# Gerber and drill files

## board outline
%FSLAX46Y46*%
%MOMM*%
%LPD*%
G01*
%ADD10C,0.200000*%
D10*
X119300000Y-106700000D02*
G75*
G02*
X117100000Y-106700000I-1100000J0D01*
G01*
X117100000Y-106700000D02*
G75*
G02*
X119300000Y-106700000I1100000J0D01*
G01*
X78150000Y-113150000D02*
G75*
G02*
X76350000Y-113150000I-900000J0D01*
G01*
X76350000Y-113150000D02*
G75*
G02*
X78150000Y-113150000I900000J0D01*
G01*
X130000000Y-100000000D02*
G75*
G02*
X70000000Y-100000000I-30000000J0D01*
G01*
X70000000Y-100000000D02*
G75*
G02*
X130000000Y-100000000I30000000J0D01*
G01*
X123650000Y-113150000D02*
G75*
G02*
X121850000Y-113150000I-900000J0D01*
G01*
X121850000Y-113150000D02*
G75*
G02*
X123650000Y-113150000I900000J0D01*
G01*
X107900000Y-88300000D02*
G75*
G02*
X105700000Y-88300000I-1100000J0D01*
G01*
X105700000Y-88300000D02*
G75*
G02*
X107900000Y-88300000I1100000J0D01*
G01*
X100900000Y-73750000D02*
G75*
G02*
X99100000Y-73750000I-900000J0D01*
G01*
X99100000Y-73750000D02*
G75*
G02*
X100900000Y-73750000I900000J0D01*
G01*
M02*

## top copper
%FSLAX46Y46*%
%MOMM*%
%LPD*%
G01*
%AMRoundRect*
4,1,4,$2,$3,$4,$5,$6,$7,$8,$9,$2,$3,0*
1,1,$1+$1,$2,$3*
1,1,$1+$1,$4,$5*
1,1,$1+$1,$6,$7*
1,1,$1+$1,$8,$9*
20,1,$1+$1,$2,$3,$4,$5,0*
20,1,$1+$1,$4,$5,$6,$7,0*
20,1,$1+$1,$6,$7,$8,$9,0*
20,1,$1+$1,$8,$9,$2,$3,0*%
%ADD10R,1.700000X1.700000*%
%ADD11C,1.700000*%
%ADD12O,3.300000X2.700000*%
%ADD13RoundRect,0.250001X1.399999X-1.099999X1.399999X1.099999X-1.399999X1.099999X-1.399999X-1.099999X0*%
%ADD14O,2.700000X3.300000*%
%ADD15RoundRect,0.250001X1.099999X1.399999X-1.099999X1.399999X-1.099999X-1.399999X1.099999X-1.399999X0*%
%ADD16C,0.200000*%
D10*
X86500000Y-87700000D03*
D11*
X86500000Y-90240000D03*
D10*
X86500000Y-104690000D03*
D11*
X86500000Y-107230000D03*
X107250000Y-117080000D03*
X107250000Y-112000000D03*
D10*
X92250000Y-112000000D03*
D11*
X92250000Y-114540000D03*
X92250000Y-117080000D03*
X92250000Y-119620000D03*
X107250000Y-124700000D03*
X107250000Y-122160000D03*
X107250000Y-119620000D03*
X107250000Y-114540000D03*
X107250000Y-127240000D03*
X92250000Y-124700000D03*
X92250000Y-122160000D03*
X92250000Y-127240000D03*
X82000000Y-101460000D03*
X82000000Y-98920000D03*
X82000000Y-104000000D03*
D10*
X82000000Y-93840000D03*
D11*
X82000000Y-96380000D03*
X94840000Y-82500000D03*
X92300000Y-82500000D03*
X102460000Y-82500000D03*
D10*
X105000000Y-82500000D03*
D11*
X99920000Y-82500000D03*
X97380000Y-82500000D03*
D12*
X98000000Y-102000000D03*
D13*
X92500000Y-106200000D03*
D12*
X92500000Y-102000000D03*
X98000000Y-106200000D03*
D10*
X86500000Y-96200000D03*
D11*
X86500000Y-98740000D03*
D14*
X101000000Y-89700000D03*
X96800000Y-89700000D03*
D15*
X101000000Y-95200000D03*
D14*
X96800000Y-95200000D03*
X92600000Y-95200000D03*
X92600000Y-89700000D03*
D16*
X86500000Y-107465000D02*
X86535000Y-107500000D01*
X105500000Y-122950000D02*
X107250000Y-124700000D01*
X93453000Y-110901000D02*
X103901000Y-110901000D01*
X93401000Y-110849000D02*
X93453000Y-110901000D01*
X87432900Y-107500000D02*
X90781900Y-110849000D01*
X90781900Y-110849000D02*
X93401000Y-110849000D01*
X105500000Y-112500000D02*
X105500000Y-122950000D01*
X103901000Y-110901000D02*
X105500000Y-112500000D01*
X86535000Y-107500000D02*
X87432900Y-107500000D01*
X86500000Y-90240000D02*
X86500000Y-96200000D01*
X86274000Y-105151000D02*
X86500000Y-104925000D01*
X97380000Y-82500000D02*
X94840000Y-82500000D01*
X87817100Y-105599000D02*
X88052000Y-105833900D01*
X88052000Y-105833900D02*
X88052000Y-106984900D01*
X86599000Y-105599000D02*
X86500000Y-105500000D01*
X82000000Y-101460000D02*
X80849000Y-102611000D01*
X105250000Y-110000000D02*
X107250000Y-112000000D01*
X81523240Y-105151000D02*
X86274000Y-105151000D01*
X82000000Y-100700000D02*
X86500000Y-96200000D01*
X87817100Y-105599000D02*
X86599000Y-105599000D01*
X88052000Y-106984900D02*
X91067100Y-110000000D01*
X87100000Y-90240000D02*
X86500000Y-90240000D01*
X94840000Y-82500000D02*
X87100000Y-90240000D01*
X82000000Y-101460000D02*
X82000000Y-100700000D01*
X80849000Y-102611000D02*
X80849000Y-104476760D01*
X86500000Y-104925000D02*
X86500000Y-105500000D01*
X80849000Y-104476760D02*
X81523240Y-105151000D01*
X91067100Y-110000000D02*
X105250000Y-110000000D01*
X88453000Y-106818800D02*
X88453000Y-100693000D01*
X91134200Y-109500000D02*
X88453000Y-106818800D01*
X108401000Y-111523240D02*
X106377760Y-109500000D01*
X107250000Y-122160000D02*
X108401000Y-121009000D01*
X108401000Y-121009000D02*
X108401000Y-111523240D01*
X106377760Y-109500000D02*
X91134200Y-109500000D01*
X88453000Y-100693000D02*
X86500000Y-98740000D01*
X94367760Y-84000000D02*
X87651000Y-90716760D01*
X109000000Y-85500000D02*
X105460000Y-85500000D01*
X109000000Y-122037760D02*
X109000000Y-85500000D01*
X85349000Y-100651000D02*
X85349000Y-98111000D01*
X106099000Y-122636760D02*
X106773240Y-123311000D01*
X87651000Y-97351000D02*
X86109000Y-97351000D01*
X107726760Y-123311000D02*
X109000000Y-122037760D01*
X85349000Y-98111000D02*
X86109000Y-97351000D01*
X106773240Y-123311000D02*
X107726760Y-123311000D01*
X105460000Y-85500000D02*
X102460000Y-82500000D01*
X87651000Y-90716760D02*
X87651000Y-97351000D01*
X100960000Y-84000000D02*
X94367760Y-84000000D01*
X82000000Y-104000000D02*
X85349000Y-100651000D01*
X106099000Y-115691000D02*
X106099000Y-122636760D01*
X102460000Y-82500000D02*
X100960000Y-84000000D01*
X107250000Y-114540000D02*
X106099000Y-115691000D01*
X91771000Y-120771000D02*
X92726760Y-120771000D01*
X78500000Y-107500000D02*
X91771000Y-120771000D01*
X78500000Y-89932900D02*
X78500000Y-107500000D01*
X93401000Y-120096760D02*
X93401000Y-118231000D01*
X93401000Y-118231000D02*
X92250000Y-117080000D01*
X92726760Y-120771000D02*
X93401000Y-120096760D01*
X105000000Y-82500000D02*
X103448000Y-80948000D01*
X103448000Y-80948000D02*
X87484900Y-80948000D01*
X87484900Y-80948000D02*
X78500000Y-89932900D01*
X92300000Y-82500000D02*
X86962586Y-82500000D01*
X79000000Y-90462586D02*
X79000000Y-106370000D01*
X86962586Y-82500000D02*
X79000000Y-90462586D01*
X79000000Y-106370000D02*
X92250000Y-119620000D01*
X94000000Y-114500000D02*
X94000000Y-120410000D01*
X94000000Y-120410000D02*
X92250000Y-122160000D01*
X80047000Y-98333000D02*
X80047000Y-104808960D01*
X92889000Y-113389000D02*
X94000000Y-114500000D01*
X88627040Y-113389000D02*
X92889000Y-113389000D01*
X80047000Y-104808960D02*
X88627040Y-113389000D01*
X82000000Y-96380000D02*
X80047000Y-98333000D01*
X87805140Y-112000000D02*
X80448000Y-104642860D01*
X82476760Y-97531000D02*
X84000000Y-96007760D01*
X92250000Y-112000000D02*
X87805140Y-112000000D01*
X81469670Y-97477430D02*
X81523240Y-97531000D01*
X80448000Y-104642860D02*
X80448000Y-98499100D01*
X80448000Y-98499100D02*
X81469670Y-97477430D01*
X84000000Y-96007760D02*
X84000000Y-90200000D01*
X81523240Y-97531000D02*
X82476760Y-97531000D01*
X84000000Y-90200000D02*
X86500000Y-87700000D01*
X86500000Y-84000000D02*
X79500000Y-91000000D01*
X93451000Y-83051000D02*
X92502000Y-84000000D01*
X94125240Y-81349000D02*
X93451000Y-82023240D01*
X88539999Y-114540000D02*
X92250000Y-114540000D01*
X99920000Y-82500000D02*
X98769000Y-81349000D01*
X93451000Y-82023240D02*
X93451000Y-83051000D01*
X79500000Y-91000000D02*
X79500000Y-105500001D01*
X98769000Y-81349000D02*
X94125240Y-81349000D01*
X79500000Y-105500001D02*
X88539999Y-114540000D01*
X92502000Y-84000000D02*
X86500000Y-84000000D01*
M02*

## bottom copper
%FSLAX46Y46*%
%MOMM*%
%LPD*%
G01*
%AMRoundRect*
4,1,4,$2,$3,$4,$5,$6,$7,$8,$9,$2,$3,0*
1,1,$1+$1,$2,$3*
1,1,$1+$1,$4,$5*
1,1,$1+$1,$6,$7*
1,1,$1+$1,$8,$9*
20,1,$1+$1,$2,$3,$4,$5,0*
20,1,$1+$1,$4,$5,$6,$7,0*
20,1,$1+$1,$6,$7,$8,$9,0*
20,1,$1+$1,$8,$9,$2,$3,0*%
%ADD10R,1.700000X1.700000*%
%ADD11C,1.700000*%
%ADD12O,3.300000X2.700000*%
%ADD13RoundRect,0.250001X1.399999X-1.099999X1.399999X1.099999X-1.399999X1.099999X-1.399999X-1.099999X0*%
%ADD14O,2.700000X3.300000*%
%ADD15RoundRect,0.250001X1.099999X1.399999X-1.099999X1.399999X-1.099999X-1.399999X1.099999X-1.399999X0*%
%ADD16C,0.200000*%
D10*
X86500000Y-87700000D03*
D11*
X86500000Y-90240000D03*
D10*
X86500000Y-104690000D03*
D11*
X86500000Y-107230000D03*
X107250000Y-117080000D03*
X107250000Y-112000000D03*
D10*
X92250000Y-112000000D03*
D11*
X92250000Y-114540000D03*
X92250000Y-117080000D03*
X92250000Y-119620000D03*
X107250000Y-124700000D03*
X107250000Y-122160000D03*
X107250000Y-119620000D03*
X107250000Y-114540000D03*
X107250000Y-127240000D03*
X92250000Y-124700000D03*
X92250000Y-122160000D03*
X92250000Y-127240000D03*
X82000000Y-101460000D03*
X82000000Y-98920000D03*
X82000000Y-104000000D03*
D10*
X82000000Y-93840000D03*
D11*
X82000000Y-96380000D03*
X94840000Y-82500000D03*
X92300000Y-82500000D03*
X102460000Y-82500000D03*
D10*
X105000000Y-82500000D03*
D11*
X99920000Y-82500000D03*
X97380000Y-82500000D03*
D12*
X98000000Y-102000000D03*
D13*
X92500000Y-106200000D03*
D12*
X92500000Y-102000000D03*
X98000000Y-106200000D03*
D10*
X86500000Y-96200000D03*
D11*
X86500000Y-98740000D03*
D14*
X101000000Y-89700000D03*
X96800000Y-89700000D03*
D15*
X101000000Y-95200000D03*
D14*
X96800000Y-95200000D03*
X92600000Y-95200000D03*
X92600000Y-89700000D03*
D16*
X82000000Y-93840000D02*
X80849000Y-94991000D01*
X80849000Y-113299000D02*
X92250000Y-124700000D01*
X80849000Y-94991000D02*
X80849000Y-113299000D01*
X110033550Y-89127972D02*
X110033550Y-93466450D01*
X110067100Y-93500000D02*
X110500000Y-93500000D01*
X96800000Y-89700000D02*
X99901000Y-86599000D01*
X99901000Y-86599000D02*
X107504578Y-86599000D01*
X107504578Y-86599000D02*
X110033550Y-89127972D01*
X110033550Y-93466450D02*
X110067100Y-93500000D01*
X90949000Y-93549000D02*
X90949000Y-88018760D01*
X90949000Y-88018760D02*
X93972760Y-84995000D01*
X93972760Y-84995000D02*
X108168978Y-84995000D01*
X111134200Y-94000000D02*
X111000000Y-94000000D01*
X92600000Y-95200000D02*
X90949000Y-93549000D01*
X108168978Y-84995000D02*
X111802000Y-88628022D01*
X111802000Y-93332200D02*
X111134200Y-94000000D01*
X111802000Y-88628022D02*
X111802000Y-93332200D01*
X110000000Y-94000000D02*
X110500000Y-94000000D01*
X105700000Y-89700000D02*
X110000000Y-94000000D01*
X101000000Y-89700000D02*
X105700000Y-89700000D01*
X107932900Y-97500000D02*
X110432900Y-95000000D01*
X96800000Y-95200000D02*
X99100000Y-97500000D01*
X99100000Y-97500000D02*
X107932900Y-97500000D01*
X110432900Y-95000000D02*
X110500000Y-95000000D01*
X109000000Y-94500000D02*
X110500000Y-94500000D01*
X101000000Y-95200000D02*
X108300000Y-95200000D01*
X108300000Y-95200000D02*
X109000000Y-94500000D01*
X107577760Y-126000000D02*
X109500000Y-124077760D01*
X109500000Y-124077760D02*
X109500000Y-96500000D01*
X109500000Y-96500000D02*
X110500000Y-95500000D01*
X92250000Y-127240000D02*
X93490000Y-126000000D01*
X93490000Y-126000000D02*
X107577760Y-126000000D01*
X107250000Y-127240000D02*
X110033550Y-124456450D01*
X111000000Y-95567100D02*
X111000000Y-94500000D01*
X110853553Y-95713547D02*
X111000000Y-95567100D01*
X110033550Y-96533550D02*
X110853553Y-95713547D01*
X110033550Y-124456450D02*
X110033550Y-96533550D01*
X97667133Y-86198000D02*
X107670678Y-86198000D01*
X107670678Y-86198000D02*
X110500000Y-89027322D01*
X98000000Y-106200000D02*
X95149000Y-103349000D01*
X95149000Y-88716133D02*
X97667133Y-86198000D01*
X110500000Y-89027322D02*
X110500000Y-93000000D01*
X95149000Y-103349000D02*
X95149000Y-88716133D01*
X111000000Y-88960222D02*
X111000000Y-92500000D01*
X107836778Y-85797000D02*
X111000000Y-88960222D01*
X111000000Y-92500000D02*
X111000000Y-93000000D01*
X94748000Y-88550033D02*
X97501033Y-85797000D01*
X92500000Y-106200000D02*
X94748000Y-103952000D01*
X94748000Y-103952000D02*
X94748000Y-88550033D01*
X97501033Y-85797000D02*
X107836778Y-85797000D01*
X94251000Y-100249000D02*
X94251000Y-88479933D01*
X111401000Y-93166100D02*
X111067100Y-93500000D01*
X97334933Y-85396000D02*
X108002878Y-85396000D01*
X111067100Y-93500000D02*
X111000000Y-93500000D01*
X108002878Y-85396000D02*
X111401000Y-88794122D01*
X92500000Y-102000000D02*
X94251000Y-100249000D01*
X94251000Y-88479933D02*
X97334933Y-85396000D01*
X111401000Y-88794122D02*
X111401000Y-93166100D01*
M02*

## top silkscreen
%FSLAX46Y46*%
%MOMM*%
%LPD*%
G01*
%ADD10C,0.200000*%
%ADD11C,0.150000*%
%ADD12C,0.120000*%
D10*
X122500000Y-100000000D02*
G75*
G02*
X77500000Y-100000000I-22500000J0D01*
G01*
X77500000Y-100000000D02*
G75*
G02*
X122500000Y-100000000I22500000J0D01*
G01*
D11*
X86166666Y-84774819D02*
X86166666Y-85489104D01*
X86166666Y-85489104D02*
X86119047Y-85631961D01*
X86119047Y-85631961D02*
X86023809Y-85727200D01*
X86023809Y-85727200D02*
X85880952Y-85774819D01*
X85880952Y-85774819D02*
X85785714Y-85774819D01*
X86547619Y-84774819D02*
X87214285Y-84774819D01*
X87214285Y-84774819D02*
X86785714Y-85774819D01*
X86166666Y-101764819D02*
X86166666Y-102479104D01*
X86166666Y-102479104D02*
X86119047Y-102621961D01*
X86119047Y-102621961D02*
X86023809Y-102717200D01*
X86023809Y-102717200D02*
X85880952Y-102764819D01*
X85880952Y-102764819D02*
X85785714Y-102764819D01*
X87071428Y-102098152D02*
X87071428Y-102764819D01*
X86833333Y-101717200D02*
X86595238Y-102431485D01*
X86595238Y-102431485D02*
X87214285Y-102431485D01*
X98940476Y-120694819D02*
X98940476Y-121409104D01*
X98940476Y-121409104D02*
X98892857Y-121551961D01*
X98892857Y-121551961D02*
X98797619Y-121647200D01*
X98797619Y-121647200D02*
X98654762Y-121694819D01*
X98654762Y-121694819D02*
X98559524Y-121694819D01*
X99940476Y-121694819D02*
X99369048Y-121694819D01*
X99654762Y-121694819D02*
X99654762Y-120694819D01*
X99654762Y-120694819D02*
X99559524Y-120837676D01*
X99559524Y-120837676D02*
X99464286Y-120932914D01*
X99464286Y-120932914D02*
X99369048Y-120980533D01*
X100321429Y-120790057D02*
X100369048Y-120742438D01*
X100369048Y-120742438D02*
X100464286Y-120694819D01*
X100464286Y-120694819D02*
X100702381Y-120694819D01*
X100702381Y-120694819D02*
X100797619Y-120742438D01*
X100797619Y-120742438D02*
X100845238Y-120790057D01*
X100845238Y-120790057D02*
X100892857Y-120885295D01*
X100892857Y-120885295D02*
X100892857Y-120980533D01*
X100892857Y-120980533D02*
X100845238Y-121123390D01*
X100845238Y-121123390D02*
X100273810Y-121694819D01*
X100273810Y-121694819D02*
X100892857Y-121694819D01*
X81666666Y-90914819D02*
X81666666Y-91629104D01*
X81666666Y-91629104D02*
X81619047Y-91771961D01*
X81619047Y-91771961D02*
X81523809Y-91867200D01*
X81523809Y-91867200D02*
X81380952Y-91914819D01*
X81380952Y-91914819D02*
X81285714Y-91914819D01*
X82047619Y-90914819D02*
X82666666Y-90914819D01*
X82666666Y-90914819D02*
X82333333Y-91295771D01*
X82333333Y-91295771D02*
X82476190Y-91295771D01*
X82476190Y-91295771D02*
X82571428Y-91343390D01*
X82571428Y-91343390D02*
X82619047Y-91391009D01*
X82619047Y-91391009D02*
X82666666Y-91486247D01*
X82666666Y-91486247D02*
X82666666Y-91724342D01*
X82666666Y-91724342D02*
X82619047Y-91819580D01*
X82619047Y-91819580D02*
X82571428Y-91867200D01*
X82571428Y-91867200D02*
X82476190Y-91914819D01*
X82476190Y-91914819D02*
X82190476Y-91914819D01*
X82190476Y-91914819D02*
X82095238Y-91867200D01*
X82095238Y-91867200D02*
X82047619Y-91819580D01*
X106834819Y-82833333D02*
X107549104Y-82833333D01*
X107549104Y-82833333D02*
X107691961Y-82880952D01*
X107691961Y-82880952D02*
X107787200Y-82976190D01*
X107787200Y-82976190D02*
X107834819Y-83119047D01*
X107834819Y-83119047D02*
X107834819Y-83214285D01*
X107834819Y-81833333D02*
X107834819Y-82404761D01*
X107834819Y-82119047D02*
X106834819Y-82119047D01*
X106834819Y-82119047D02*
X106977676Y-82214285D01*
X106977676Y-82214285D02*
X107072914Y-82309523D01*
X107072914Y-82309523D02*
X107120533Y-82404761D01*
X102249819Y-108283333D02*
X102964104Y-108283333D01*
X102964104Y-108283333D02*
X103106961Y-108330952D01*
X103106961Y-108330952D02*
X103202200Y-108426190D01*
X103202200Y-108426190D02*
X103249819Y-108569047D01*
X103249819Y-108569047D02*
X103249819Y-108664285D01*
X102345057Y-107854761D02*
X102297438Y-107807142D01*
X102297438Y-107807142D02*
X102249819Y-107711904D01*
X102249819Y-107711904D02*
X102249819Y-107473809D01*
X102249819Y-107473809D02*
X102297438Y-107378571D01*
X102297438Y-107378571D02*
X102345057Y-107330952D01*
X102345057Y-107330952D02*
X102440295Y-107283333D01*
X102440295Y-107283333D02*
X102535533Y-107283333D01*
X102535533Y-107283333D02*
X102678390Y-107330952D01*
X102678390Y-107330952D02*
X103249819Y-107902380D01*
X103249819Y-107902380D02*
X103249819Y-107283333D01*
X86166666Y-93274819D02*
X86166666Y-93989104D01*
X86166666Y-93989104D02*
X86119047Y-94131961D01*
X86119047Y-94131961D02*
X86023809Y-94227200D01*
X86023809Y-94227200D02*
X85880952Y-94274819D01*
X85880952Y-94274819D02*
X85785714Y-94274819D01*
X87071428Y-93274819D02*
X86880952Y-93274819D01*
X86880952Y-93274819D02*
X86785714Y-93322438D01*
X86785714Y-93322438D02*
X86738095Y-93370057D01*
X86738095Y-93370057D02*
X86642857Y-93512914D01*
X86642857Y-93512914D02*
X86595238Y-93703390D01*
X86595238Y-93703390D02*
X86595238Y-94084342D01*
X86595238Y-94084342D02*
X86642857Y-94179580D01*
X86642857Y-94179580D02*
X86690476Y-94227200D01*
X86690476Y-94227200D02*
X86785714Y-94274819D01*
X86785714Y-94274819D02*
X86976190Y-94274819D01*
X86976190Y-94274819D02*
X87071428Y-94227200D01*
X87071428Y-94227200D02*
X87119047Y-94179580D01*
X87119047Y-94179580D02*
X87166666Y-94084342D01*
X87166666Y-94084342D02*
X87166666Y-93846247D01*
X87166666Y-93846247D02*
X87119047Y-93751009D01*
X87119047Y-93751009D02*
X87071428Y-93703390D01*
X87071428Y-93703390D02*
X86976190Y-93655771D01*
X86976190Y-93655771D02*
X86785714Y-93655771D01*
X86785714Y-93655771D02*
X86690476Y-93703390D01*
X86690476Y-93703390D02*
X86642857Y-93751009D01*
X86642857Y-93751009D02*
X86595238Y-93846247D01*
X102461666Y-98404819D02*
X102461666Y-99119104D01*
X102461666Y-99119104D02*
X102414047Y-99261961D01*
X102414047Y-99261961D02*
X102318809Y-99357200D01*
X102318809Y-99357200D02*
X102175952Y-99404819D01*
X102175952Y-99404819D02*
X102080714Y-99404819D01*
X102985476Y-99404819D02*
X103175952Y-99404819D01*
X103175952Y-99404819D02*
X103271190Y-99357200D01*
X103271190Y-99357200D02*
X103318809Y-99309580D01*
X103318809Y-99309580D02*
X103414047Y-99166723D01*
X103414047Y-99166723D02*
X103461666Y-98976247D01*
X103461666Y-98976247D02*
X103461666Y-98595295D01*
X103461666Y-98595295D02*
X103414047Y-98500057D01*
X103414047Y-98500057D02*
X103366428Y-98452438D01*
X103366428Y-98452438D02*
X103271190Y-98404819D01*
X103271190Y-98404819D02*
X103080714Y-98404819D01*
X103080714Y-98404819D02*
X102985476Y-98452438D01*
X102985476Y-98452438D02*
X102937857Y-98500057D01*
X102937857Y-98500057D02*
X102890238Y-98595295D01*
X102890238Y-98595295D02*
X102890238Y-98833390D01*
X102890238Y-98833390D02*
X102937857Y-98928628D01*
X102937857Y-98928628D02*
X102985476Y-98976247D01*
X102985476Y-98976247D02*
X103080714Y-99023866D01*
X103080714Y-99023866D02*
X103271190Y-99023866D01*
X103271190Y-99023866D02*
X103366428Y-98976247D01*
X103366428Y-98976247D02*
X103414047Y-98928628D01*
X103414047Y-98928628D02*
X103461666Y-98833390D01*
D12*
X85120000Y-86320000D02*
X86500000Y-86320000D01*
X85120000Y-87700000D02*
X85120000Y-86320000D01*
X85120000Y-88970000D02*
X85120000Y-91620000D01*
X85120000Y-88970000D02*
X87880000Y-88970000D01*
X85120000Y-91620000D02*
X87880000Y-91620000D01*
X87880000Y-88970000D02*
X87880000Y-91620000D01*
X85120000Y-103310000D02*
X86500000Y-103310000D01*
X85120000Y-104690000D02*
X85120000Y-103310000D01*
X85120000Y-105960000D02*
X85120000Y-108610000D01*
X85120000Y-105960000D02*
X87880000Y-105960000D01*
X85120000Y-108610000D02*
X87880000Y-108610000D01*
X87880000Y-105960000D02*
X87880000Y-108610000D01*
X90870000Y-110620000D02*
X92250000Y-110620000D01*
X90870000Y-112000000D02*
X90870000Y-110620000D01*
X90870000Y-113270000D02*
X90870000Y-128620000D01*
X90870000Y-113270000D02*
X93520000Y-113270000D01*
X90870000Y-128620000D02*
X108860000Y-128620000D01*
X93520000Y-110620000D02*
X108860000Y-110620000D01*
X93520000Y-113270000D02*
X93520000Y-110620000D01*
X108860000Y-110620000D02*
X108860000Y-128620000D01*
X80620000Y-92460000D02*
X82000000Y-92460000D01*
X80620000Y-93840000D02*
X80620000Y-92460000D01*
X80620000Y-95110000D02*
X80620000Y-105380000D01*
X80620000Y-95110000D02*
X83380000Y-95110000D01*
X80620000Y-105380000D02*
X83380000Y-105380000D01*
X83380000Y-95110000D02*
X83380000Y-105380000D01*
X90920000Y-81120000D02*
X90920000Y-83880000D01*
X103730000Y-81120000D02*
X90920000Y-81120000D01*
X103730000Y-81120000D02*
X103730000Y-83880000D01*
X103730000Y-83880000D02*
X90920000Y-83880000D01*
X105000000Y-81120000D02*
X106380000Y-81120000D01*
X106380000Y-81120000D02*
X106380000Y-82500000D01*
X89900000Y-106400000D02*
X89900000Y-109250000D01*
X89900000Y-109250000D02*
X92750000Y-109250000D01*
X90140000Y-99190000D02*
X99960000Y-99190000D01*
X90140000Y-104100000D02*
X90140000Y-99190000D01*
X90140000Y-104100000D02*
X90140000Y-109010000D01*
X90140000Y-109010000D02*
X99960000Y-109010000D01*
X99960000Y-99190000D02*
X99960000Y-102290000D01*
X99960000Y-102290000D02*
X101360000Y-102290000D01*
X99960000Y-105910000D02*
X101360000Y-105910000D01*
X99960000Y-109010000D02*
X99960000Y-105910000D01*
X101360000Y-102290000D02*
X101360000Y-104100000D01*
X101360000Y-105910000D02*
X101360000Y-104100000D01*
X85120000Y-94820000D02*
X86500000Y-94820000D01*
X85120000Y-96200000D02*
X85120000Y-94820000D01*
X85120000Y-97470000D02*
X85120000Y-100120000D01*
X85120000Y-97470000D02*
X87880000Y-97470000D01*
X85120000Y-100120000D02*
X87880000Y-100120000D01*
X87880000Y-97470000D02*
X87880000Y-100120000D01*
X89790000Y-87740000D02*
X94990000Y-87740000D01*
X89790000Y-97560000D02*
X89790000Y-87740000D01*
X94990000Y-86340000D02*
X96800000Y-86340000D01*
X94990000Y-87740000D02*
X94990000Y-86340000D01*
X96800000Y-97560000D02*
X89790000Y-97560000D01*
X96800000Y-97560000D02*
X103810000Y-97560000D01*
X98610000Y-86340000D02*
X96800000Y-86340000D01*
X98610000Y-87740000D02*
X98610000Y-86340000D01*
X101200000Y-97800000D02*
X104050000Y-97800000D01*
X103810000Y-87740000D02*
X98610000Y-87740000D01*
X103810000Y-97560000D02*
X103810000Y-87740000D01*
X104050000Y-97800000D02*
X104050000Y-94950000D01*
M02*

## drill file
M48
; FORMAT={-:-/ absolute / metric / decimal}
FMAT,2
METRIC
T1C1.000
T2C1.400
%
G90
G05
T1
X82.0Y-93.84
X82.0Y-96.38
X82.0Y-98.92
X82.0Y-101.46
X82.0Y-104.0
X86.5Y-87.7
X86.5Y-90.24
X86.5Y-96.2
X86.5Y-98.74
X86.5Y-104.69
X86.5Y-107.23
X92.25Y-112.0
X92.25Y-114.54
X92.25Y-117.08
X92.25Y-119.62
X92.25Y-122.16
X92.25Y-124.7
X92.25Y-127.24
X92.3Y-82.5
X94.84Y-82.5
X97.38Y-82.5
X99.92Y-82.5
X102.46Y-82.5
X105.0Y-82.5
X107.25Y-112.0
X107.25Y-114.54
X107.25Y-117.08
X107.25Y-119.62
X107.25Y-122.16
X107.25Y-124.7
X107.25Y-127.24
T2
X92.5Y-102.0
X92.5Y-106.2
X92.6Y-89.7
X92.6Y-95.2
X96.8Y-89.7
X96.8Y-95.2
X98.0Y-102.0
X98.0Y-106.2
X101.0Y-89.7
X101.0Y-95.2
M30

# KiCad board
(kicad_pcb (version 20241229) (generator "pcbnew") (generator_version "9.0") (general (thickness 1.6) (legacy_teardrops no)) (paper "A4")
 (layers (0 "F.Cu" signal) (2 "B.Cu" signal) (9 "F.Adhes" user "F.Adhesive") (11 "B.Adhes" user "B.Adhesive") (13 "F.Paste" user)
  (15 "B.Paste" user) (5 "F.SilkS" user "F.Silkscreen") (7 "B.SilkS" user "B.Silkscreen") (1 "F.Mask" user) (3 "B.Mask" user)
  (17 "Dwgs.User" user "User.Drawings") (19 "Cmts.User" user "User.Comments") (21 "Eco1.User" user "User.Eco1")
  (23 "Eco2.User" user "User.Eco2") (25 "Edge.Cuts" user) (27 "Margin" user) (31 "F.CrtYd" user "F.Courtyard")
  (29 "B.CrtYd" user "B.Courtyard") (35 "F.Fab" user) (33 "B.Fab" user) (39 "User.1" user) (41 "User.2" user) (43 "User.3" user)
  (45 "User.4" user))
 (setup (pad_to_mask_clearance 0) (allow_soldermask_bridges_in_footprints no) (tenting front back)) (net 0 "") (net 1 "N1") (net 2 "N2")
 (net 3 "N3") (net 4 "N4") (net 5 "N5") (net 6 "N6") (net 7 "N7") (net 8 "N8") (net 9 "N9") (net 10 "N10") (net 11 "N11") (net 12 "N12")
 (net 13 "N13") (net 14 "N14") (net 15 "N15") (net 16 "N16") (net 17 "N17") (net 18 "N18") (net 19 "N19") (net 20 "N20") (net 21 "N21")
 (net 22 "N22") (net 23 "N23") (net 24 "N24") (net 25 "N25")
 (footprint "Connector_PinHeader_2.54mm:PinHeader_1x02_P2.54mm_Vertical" (layer "F.Cu") (at 86.5 87.7)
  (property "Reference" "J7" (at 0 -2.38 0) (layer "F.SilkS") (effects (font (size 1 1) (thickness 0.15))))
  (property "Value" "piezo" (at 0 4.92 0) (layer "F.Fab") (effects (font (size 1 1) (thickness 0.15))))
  (fp_line (start -1.38 -1.38) (end 0 -1.38) (stroke (width 0.12) (type solid)) (layer "F.SilkS"))
  (fp_line (start -1.38 0) (end -1.38 -1.38) (stroke (width 0.12) (type solid)) (layer "F.SilkS"))
  (fp_line (start -1.38 1.27) (end -1.38 3.92) (stroke (width 0.12) (type solid)) (layer "F.SilkS"))
  (fp_line (start -1.38 1.27) (end 1.38 1.27) (stroke (width 0.12) (type solid)) (layer "F.SilkS"))
  (fp_line (start -1.38 3.92) (end 1.38 3.92) (stroke (width 0.12) (type solid)) (layer "F.SilkS"))
  (fp_line (start 1.38 1.27) (end 1.38 3.92) (stroke (width 0.12) (type solid)) (layer "F.SilkS"))
  (pad "1" thru_hole rect (at 0 0) (size 1.7 1.7) (drill 1) (layers "*.Cu" "*.Mask") (remove_unused_layers no) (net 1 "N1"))
  (pad "2" thru_hole circle (at 0 2.54) (size 1.7 1.7) (drill 1) (layers "*.Cu" "*.Mask") (remove_unused_layers no) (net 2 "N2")))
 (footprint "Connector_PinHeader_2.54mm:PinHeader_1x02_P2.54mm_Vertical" (layer "F.Cu") (at 86.5 104.69)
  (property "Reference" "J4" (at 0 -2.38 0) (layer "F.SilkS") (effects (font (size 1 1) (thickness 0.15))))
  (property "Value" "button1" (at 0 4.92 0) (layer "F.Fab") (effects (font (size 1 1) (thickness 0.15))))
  (fp_line (start -1.38 -1.38) (end 0 -1.38) (stroke (width 0.12) (type solid)) (layer "F.SilkS"))
  (fp_line (start -1.38 0) (end -1.38 -1.38) (stroke (width 0.12) (type solid)) (layer "F.SilkS"))
  (fp_line (start -1.38 1.27) (end -1.38 3.92) (stroke (width 0.12) (type solid)) (layer "F.SilkS"))
  (fp_line (start -1.38 1.27) (end 1.38 1.27) (stroke (width 0.12) (type solid)) (layer "F.SilkS"))
  (fp_line (start -1.38 3.92) (end 1.38 3.92) (stroke (width 0.12) (type solid)) (layer "F.SilkS"))
  (fp_line (start 1.38 1.27) (end 1.38 3.92) (stroke (width 0.12) (type solid)) (layer "F.SilkS"))
  (pad "1" thru_hole rect (at 0 0) (size 1.7 1.7) (drill 1) (layers "*.Cu" "*.Mask") (remove_unused_layers no) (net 2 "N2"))
  (pad "2" thru_hole circle (at 0 2.54) (size 1.7 1.7) (drill 1) (layers "*.Cu" "*.Mask") (remove_unused_layers no) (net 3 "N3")))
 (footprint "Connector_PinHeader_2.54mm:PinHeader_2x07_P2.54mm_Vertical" (layer "F.Cu") (at 92.25 112)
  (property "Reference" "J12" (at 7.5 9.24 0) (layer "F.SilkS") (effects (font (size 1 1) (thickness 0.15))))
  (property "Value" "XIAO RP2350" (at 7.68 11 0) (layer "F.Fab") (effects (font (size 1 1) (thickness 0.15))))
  (fp_line (start -1.38 -1.38) (end 0 -1.38) (stroke (width 0.12) (type solid)) (layer "F.SilkS"))
  (fp_line (start -1.38 0) (end -1.38 -1.38) (stroke (width 0.12) (type solid)) (layer "F.SilkS"))
  (fp_line (start -1.38 1.27) (end -1.38 16.62) (stroke (width 0.12) (type solid)) (layer "F.SilkS"))
  (fp_line (start -1.38 1.27) (end 1.27 1.27) (stroke (width 0.12) (type solid)) (layer "F.SilkS"))
  (fp_line (start -1.38 16.62) (end 16.61 16.62) (stroke (width 0.12) (type solid)) (layer "F.SilkS"))
  (fp_line (start 1.27 -1.38) (end 16.61 -1.38) (stroke (width 0.12) (type solid)) (layer "F.SilkS"))
  (fp_line (start 1.27 1.27) (end 1.27 -1.38) (stroke (width 0.12) (type solid)) (layer "F.SilkS"))
  (fp_line (start 16.61 -1.38) (end 16.61 16.62) (stroke (width 0.12) (type solid)) (layer "F.SilkS"))
  (pad "3V3" thru_hole circle (at 15 5.08) (size 1.7 1.7) (drill 1) (layers "*.Cu" "*.Mask") (remove_unused_layers no) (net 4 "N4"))
  (pad "5V" thru_hole circle (at 15 0) (size 1.7 1.7) (drill 1) (layers "*.Cu" "*.Mask") (remove_unused_layers no) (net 2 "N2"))
  (pad "A0" thru_hole rect (at 0 0) (size 1.7 1.7) (drill 1) (layers "*.Cu" "*.Mask") (remove_unused_layers no) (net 1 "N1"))
  (pad "A1" thru_hole circle (at 0 2.54) (size 1.7 1.7) (drill 1) (layers "*.Cu" "*.Mask") (remove_unused_layers no) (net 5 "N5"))
  (pad "A2" thru_hole circle (at 0 5.08) (size 1.7 1.7) (drill 1) (layers "*.Cu" "*.Mask") (remove_unused_layers no) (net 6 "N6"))
  (pad "D3" thru_hole circle (at 0 7.62) (size 1.7 1.7) (drill 1) (layers "*.Cu" "*.Mask") (remove_unused_layers no) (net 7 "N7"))
  (pad "D8" thru_hole circle (at 15 12.7) (size 1.7 1.7) (drill 1) (layers "*.Cu" "*.Mask") (remove_unused_layers no) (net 3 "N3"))
  (pad "D9" thru_hole circle (at 15 10.16) (size 1.7 1.7) (drill 1) (layers "*.Cu" "*.Mask") (remove_unused_layers no) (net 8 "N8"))
  (pad "D10" thru_hole circle (at 15 7.62) (size 1.7 1.7) (drill 1) (layers "*.Cu" "*.Mask") (remove_unused_layers no) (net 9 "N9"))
  (pad "GND" thru_hole circle (at 15 2.54) (size 1.7 1.7) (drill 1) (layers "*.Cu" "*.Mask") (remove_unused_layers no) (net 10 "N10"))
  (pad "RX0" thru_hole circle (at 15 15.24) (size 1.7 1.7) (drill 1) (layers "*.Cu" "*.Mask") (remove_unused_layers no) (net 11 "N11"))
  (pad "SCL1" thru_hole circle (at 0 12.7) (size 1.7 1.7) (drill 1) (layers "*.Cu" "*.Mask") (remove_unused_layers no) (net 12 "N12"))
  (pad "SDA1" thru_hole circle (at 0 10.16) (size 1.7 1.7) (drill 1) (layers "*.Cu" "*.Mask") (remove_unused_layers no) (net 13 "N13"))
  (pad "TX0" thru_hole circle (at 0 15.24) (size 1.7 1.7) (drill 1) (layers "*.Cu" "*.Mask") (remove_unused_layers no) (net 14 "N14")))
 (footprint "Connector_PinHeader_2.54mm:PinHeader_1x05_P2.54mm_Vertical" (layer "F.Cu") (at 82 93.84)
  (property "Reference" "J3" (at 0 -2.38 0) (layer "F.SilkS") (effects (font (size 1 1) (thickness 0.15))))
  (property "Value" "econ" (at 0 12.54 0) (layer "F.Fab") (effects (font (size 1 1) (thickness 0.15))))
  (fp_line (start -1.38 -1.38) (end 0 -1.38) (stroke (width 0.12) (type solid)) (layer "F.SilkS"))
  (fp_line (start -1.38 0) (end -1.38 -1.38) (stroke (width 0.12) (type solid)) (layer "F.SilkS"))
  (fp_line (start -1.38 1.27) (end -1.38 11.54) (stroke (width 0.12) (type solid)) (layer "F.SilkS"))
  (fp_line (start -1.38 1.27) (end 1.38 1.27) (stroke (width 0.12) (type solid)) (layer "F.SilkS"))
  (fp_line (start -1.38 11.54) (end 1.38 11.54) (stroke (width 0.12) (type solid)) (layer "F.SilkS"))
  (fp_line (start 1.38 1.27) (end 1.38 11.54) (stroke (width 0.12) (type solid)) (layer "F.SilkS"))
  (pad "5v" thru_hole circle (at 0 7.62) (size 1.7 1.7) (drill 1) (layers "*.Cu" "*.Mask") (remove_unused_layers no) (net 2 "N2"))
  (pad "18v" thru_hole circle (at 0 5.08) (size 1.7 1.7) (drill 1) (layers "*.Cu" "*.Mask") (remove_unused_layers no) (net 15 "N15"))
  (pad "GND" thru_hole circle (at 0 10.16) (size 1.7 1.7) (drill 1) (layers "*.Cu" "*.Mask") (remove_unused_layers no) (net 10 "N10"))
  (pad "SCL" thru_hole rect (at 0 0) (size 1.7 1.7) (drill 1) (layers "*.Cu" "*.Mask") (remove_unused_layers no) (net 12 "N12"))
  (pad "SDA" thru_hole circle (at 0 2.54) (size 1.7 1.7) (drill 1) (layers "*.Cu" "*.Mask") (remove_unused_layers no) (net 13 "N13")))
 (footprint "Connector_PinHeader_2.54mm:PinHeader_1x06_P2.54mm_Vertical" (layer "F.Cu") (at 105 82.5 -90)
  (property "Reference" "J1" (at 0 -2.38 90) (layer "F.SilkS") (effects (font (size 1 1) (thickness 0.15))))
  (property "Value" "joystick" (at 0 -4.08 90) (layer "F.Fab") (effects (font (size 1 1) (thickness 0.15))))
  (fp_line (start -1.38 14.08) (end 1.38 14.08) (stroke (width 0.12) (type solid)) (layer "F.SilkS"))
  (fp_line (start -1.38 1.27) (end -1.38 14.08) (stroke (width 0.12) (type solid)) (layer "F.SilkS"))
  (fp_line (start -1.38 1.27) (end 1.38 1.27) (stroke (width 0.12) (type solid)) (layer "F.SilkS"))
  (fp_line (start 1.38 1.27) (end 1.38 14.08) (stroke (width 0.12) (type solid)) (layer "F.SilkS"))
  (fp_line (start -1.38 0) (end -1.38 -1.38) (stroke (width 0.12) (type solid)) (layer "F.SilkS"))
  (fp_line (start -1.38 -1.38) (end 0 -1.38) (stroke (width 0.12) (type solid)) (layer "F.SilkS"))
  (pad "B0" thru_hole circle (at 0 10.16 270) (size 1.7 1.7) (drill 1) (layers "*.Cu" "*.Mask") (remove_unused_layers no) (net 2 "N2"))
  (pad "B1" thru_hole circle (at 0 12.7 270) (size 1.7 1.7) (drill 1) (layers "*.Cu" "*.Mask") (remove_unused_layers no) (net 7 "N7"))
  (pad "GND" thru_hole circle (at 0 2.54 270) (size 1.7 1.7) (drill 1) (layers "*.Cu" "*.Mask") (remove_unused_layers no) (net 10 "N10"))
  (pad "LR" thru_hole rect (at 0 0 270) (size 1.7 1.7) (drill 1) (layers "*.Cu" "*.Mask" "F.Adhes") (remove_unused_layers no) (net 6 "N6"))
  (pad "UD" thru_hole circle (at 0 5.08 270) (size 1.7 1.7) (drill 1) (layers "*.Cu" "*.Mask") (remove_unused_layers no) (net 5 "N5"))
  (pad "VCC" thru_hole circle (at 0 7.62 270) (size 1.7 1.7) (drill 1) (layers "*.Cu" "*.Mask") (remove_unused_layers no) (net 2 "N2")))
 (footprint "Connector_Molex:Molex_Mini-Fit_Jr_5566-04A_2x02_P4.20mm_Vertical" (layer "F.Cu") (at 92.5 106.2 90)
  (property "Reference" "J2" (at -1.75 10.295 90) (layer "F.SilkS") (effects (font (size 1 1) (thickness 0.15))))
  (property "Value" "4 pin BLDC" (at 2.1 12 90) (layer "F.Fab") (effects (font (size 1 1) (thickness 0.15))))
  (fp_line (start -0.2 -2.6) (end -3.05 -2.6) (stroke (width 0.12) (type solid)) (layer "F.SilkS"))
  (fp_line (start -3.05 -2.6) (end -3.05 0.25) (stroke (width 0.12) (type solid)) (layer "F.SilkS"))
  (fp_line (start 7.01 -2.36) (end 7.01 7.46) (stroke (width 0.12) (type solid)) (layer "F.SilkS"))
  (fp_line (start 2.1 -2.36) (end 7.01 -2.36) (stroke (width 0.12) (type solid)) (layer "F.SilkS"))
  (fp_line (start 2.1 -2.36) (end -2.81 -2.36) (stroke (width 0.12) (type solid)) (layer "F.SilkS"))
  (fp_line (start -2.81 -2.36) (end -2.81 7.46) (stroke (width 0.12) (type solid)) (layer "F.SilkS"))
  (fp_line (start 7.01 7.46) (end 3.91 7.46) (stroke (width 0.12) (type solid)) (layer "F.SilkS"))
  (fp_line (start 3.91 7.46) (end 3.91 8.86) (stroke (width 0.12) (type solid)) (layer "F.SilkS"))
  (fp_line (start 0.29 7.46) (end 0.29 8.86) (stroke (width 0.12) (type solid)) (layer "F.SilkS"))
  (fp_line (start -2.81 7.46) (end 0.29 7.46) (stroke (width 0.12) (type solid)) (layer "F.SilkS"))
  (fp_line (start 3.91 8.86) (end 2.1 8.86) (stroke (width 0.12) (type solid)) (layer "F.SilkS"))
  (fp_line (start 0.29 8.86) (end 2.1 8.86) (stroke (width 0.12) (type solid)) (layer "F.SilkS"))
  (pad "nc" thru_hole oval (at 4.2 5.5 90) (size 2.7 3.3) (drill 1.4) (layers "*.Cu" "*.Mask") (remove_unused_layers no) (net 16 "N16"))
  (pad "w1" thru_hole roundrect (at 0 0 90) (size 2.7 3.3) (drill 1.4) (layers "*.Cu" "*.Mask") (remove_unused_layers no)
   (roundrect_rratio 0.092593) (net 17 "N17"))
  (pad "w2" thru_hole oval (at 4.2 0 90) (size 2.7 3.3) (drill 1.4) (layers "*.Cu" "*.Mask") (remove_unused_layers no) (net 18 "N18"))
  (pad "w3" thru_hole oval (at 0 5.5 90) (size 2.7 3.3) (drill 1.4) (layers "*.Cu" "*.Mask") (remove_unused_layers no) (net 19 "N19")))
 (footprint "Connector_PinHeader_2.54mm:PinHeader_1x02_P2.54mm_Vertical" (layer "F.Cu") (at 86.5 96.2)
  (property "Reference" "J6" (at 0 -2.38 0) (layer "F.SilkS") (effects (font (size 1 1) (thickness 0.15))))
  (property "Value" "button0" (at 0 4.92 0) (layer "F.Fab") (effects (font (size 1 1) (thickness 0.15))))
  (fp_line (start -1.38 -1.38) (end 0 -1.38) (stroke (width 0.12) (type solid)) (layer "F.SilkS"))
  (fp_line (start -1.38 0) (end -1.38 -1.38) (stroke (width 0.12) (type solid)) (layer "F.SilkS"))
  (fp_line (start -1.38 1.27) (end -1.38 3.92) (stroke (width 0.12) (type solid)) (layer "F.SilkS"))
  (fp_line (start -1.38 1.27) (end 1.38 1.27) (stroke (width 0.12) (type solid)) (layer "F.SilkS"))
  (fp_line (start -1.38 3.92) (end 1.38 3.92) (stroke (width 0.12) (type solid)) (layer "F.SilkS"))
  (fp_line (start 1.38 1.27) (end 1.38 3.92) (stroke (width 0.12) (type solid)) (layer "F.SilkS"))
  (pad "1" thru_hole rect (at 0 0) (size 1.7 1.7) (drill 1) (layers "*.Cu" "*.Mask") (remove_unused_layers no) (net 2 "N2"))
  (pad "2" thru_hole circle (at 0 2.54) (size 1.7 1.7) (drill 1) (layers "*.Cu" "*.Mask") (remove_unused_layers no) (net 8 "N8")))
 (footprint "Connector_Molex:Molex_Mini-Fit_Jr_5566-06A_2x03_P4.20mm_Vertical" (layer "F.Cu") (at 101 95.2 180)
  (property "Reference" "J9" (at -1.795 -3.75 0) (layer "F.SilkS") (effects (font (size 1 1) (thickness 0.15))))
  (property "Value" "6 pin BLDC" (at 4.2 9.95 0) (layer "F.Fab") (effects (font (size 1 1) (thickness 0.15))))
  (fp_line (start 11.21 7.46) (end 6.01 7.46) (stroke (width 0.12) (type solid)) (layer "F.SilkS"))
  (fp_line (start 11.21 -2.36) (end 11.21 7.46) (stroke (width 0.12) (type solid)) (layer "F.SilkS"))
  (fp_line (start 6.01 8.86) (end 4.2 8.86) (stroke (width 0.12) (type solid)) (layer "F.SilkS"))
  (fp_line (start 6.01 7.46) (end 6.01 8.86) (stroke (width 0.12) (type solid)) (layer "F.SilkS"))
  (fp_line (start 4.2 -2.36) (end 11.21 -2.36) (stroke (width 0.12) (type solid)) (layer "F.SilkS"))
  (fp_line (start 4.2 -2.36) (end -2.81 -2.36) (stroke (width 0.12) (type solid)) (layer "F.SilkS"))
  (fp_line (start 2.39 8.86) (end 4.2 8.86) (stroke (width 0.12) (type solid)) (layer "F.SilkS"))
  (fp_line (start 2.39 7.46) (end 2.39 8.86) (stroke (width 0.12) (type solid)) (layer "F.SilkS"))
  (fp_line (start -0.2 -2.6) (end -3.05 -2.6) (stroke (width 0.12) (type solid)) (layer "F.SilkS"))
  (fp_line (start -2.81 7.46) (end 2.39 7.46) (stroke (width 0.12) (type solid)) (layer "F.SilkS"))
  (fp_line (start -2.81 -2.36) (end -2.81 7.46) (stroke (width 0.12) (type solid)) (layer "F.SilkS"))
  (fp_line (start -3.05 -2.6) (end -3.05 0.25) (stroke (width 0.12) (type solid)) (layer "F.SilkS"))
  (pad "GND" thru_hole oval (at 0 5.5 180) (size 2.7 3.3) (drill 1.4) (layers "*.Cu" "*.Mask") (remove_unused_layers no) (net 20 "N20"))
  (pad "Vh" thru_hole oval (at 4.2 5.5 180) (size 2.7 3.3) (drill 1.4) (layers "*.Cu" "*.Mask") (remove_unused_layers no) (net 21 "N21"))
  (pad "h1" thru_hole roundrect (at 0 0 180) (size 2.7 3.3) (drill 1.4) (layers "*.Cu" "*.Mask") (remove_unused_layers no)
   (roundrect_rratio 0.092593) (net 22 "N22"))
  (pad "h2" thru_hole oval (at 4.2 0 180) (size 2.7 3.3) (drill 1.4) (layers "*.Cu" "*.Mask") (remove_unused_layers no) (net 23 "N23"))
  (pad "h3" thru_hole oval (at 8.4 0 180) (size 2.7 3.3) (drill 1.4) (layers "*.Cu" "*.Mask") (remove_unused_layers no) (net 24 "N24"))
  (pad "nc" thru_hole oval (at 8.4 5.5 180) (size 2.7 3.3) (drill 1.4) (layers "*.Cu" "*.Mask") (remove_unused_layers no) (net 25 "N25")))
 (gr_circle (center 100 100) (end 122.5 100) (stroke (width 0.2) (type solid)) (fill no) (layer "F.SilkS"))
 (gr_circle (center 118.2 106.7) (end 119.3 106.7) (stroke (width 0.2) (type solid)) (fill no) (layer "Edge.Cuts"))
 (gr_circle (center 77.25 113.15) (end 78.15 113.15) (stroke (width 0.2) (type solid)) (fill no) (layer "Edge.Cuts"))
 (gr_circle (center 100 100) (end 130 100) (stroke (width 0.2) (type solid)) (fill no) (locked yes) (layer "Edge.Cuts"))
 (gr_circle (center 122.75 113.15) (end 123.65 113.15) (stroke (width 0.2) (type solid)) (fill no) (layer "Edge.Cuts"))
 (gr_circle (center 106.8 88.3) (end 107.9 88.3) (stroke (width 0.2) (type solid)) (fill no) (layer "Edge.Cuts"))
 (gr_circle (center 100 73.75) (end 100.9 73.75) (stroke (width 0.2) (type solid)) (fill no) (layer "Edge.Cuts"))
 (segment (start 86.5 107.465) (end 86.535 107.5) (width 0.2) (layer "F.Cu") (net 3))
 (segment (start 105.5 122.95) (end 107.25 124.7) (width 0.2) (layer "F.Cu") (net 3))
 (segment (start 93.453 110.901) (end 103.901 110.901) (width 0.2) (layer "F.Cu") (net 3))
 (segment (start 93.401 110.849) (end 93.453 110.901) (width 0.2) (layer "F.Cu") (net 3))
 (segment (start 87.4329 107.5) (end 90.7819 110.849) (width 0.2) (layer "F.Cu") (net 3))
 (segment (start 90.7819 110.849) (end 93.401 110.849) (width 0.2) (layer "F.Cu") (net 3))
 (segment (start 105.5 112.5) (end 105.5 122.95) (width 0.2) (layer "F.Cu") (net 3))
 (segment (start 103.901 110.901) (end 105.5 112.5) (width 0.2) (layer "F.Cu") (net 3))
 (segment (start 86.535 107.5) (end 87.4329 107.5) (width 0.2) (layer "F.Cu") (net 3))
 (segment (start 86.5 90.24) (end 86.5 96.2) (width 0.2) (layer "F.Cu") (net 2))
 (segment (start 86.274 105.151) (end 86.5 104.925) (width 0.2) (layer "F.Cu") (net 2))
 (segment (start 97.38 82.5) (end 94.84 82.5) (width 0.2) (layer "F.Cu") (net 2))
 (segment (start 87.8171 105.599) (end 88.052 105.8339) (width 0.2) (layer "F.Cu") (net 2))
 (segment (start 88.052 105.8339) (end 88.052 106.9849) (width 0.2) (layer "F.Cu") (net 2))
 (segment (start 86.599 105.599) (end 86.5 105.5) (width 0.2) (layer "F.Cu") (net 2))
 (segment (start 82 101.46) (end 80.849 102.611) (width 0.2) (layer "F.Cu") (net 2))
 (segment (start 105.25 110) (end 107.25 112) (width 0.2) (layer "F.Cu") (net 2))
 (segment (start 81.52324 105.151) (end 86.274 105.151) (width 0.2) (layer "F.Cu") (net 2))
 (segment (start 82 100.7) (end 86.5 96.2) (width 0.2) (layer "F.Cu") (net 2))
 (segment (start 87.8171 105.599) (end 86.599 105.599) (width 0.2) (layer "F.Cu") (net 2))
 (segment (start 88.052 106.9849) (end 91.0671 110) (width 0.2) (layer "F.Cu") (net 2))
 (segment (start 87.1 90.24) (end 86.5 90.24) (width 0.2) (layer "F.Cu") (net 2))
 (segment (start 94.84 82.5) (end 87.1 90.24) (width 0.2) (layer "F.Cu") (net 2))
 (segment (start 82 101.46) (end 82 100.7) (width 0.2) (layer "F.Cu") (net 2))
 (segment (start 80.849 102.611) (end 80.849 104.47676) (width 0.2) (layer "F.Cu") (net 2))
 (segment (start 86.5 104.925) (end 86.5 105.5) (width 0.2) (layer "F.Cu") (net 2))
 (segment (start 80.849 104.47676) (end 81.52324 105.151) (width 0.2) (layer "F.Cu") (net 2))
 (segment (start 91.0671 110) (end 105.25 110) (width 0.2) (layer "F.Cu") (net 2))
 (segment (start 88.453 106.8188) (end 88.453 100.693) (width 0.2) (layer "F.Cu") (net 8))
 (segment (start 91.1342 109.5) (end 88.453 106.8188) (width 0.2) (layer "F.Cu") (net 8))
 (segment (start 108.401 111.52324) (end 106.37776 109.5) (width 0.2) (layer "F.Cu") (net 8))
 (segment (start 107.25 122.16) (end 108.401 121.009) (width 0.2) (layer "F.Cu") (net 8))
 (segment (start 108.401 121.009) (end 108.401 111.52324) (width 0.2) (layer "F.Cu") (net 8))
 (segment (start 106.37776 109.5) (end 91.1342 109.5) (width 0.2) (layer "F.Cu") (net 8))
 (segment (start 88.453 100.693) (end 86.5 98.74) (width 0.2) (layer "F.Cu") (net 8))
 (segment (start 94.36776 84) (end 87.651 90.71676) (width 0.2) (layer "F.Cu") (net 10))
 (segment (start 109 85.5) (end 105.46 85.5) (width 0.2) (layer "F.Cu") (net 10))
 (segment (start 109 122.03776) (end 109 85.5) (width 0.2) (layer "F.Cu") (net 10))
 (segment (start 85.349 100.651) (end 85.349 98.111) (width 0.2) (layer "F.Cu") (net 10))
 (segment (start 106.099 122.63676) (end 106.77324 123.311) (width 0.2) (layer "F.Cu") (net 10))
 (segment (start 87.651 97.351) (end 86.109 97.351) (width 0.2) (layer "F.Cu") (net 10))
 (segment (start 107.72676 123.311) (end 109 122.03776) (width 0.2) (layer "F.Cu") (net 10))
 (segment (start 85.349 98.111) (end 86.109 97.351) (width 0.2) (layer "F.Cu") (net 10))
 (segment (start 106.77324 123.311) (end 107.72676 123.311) (width 0.2) (layer "F.Cu") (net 10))
 (segment (start 105.46 85.5) (end 102.46 82.5) (width 0.2) (layer "F.Cu") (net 10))
 (segment (start 87.651 90.71676) (end 87.651 97.351) (width 0.2) (layer "F.Cu") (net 10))
 (segment (start 100.96 84) (end 94.36776 84) (width 0.2) (layer "F.Cu") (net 10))
 (segment (start 82 104) (end 85.349 100.651) (width 0.2) (layer "F.Cu") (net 10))
 (segment (start 106.099 115.691) (end 106.099 122.63676) (width 0.2) (layer "F.Cu") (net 10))
 (segment (start 102.46 82.5) (end 100.96 84) (width 0.2) (layer "F.Cu") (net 10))
 (segment (start 107.25 114.54) (end 106.099 115.691) (width 0.2) (layer "F.Cu") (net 10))
 (segment (start 91.771 120.771) (end 92.72676 120.771) (width 0.2) (layer "F.Cu") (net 6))
 (segment (start 78.5 107.5) (end 91.771 120.771) (width 0.2) (layer "F.Cu") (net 6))
 (segment (start 78.5 89.9329) (end 78.5 107.5) (width 0.2) (layer "F.Cu") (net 6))
 (segment (start 93.401 120.09676) (end 93.401 118.231) (width 0.2) (layer "F.Cu") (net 6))
 (segment (start 93.401 118.231) (end 92.25 117.08) (width 0.2) (layer "F.Cu") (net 6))
 (segment (start 92.72676 120.771) (end 93.401 120.09676) (width 0.2) (layer "F.Cu") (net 6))
 (segment (start 105 82.5) (end 103.448 80.948) (width 0.2) (layer "F.Cu") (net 6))
 (segment (start 103.448 80.948) (end 87.4849 80.948) (width 0.2) (layer "F.Cu") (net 6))
 (segment (start 87.4849 80.948) (end 78.5 89.9329) (width 0.2) (layer "F.Cu") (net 6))
 (segment (start 92.3 82.5) (end 86.962586 82.5) (width 0.2) (layer "F.Cu") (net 7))
 (segment (start 79 90.462586) (end 79 106.37) (width 0.2) (layer "F.Cu") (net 7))
 (segment (start 86.962586 82.5) (end 79 90.462586) (width 0.2) (layer "F.Cu") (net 7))
 (segment (start 79 106.37) (end 92.25 119.62) (width 0.2) (layer "F.Cu") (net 7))
 (segment (start 82 93.84) (end 80.849 94.991) (width 0.2) (layer "B.Cu") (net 12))
 (segment (start 80.849 113.299) (end 92.25 124.7) (width 0.2) (layer "B.Cu") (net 12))
 (segment (start 80.849 94.991) (end 80.849 113.299) (width 0.2) (layer "B.Cu") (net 12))
 (segment (start 94 114.5) (end 94 120.41) (width 0.2) (layer "F.Cu") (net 13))
 (segment (start 94 120.41) (end 92.25 122.16) (width 0.2) (layer "F.Cu") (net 13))
 (segment (start 80.047 98.333) (end 80.047 104.80896) (width 0.2) (layer "F.Cu") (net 13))
 (segment (start 92.889 113.389) (end 94 114.5) (width 0.2) (layer "F.Cu") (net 13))
 (segment (start 88.62704 113.389) (end 92.889 113.389) (width 0.2) (layer "F.Cu") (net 13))
 (segment (start 80.047 104.80896) (end 88.62704 113.389) (width 0.2) (layer "F.Cu") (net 13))
 (segment (start 82 96.38) (end 80.047 98.333) (width 0.2) (layer "F.Cu") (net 13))
 (segment (start 87.80514 112) (end 80.448 104.64286) (width 0.2) (layer "F.Cu") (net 1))
 (segment (start 82.47676 97.531) (end 84 96.00776) (width 0.2) (layer "F.Cu") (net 1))
 (segment (start 92.25 112) (end 87.80514 112) (width 0.2) (layer "F.Cu") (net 1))
 (segment (start 81.46967 97.47743) (end 81.52324 97.531) (width 0.2) (layer "F.Cu") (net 1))
 (segment (start 80.448 104.64286) (end 80.448 98.4991) (width 0.2) (layer "F.Cu") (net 1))
 (segment (start 80.448 98.4991) (end 81.46967 97.47743) (width 0.2) (layer "F.Cu") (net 1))
 (segment (start 84 96.00776) (end 84 90.2) (width 0.2) (layer "F.Cu") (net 1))
 (segment (start 81.52324 97.531) (end 82.47676 97.531) (width 0.2) (layer "F.Cu") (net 1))
 (segment (start 84 90.2) (end 86.5 87.7) (width 0.2) (layer "F.Cu") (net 1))
 (segment (start 110.03355 89.127972) (end 110.03355 93.46645) (width 0.2) (layer "B.Cu") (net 21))
 (segment (start 110.0671 93.5) (end 110.5 93.5) (width 0.2) (layer "B.Cu") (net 21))
 (segment (start 96.8 89.7) (end 99.901 86.599) (width 0.2) (layer "B.Cu") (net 21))
 (segment (start 99.901 86.599) (end 107.504578 86.599) (width 0.2) (layer "B.Cu") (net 21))
 (segment (start 107.504578 86.599) (end 110.03355 89.127972) (width 0.2) (layer "B.Cu") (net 21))
 (segment (start 110.03355 93.46645) (end 110.0671 93.5) (width 0.2) (layer "B.Cu") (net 21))
 (segment (start 90.949 93.549) (end 90.949 88.01876) (width 0.2) (layer "B.Cu") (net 24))
 (segment (start 90.949 88.01876) (end 93.97276 84.995) (width 0.2) (layer "B.Cu") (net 24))
 (segment (start 93.97276 84.995) (end 108.168978 84.995) (width 0.2) (layer "B.Cu") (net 24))
 (segment (start 111.1342 94) (end 111 94) (width 0.2) (layer "B.Cu") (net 24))
 (segment (start 92.6 95.2) (end 90.949 93.549) (width 0.2) (layer "B.Cu") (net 24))
 (segment (start 108.168978 84.995) (end 111.802 88.628022) (width 0.2) (layer "B.Cu") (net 24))
 (segment (start 111.802 93.3322) (end 111.1342 94) (width 0.2) (layer "B.Cu") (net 24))
 (segment (start 111.802 88.628022) (end 111.802 93.3322) (width 0.2) (layer "B.Cu") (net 24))
 (segment (start 110 94) (end 110.5 94) (width 0.2) (layer "B.Cu") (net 20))
 (segment (start 105.7 89.7) (end 110 94) (width 0.2) (layer "B.Cu") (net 20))
 (segment (start 101 89.7) (end 105.7 89.7) (width 0.2) (layer "B.Cu") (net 20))
 (segment (start 107.9329 97.5) (end 110.4329 95) (width 0.2) (layer "B.Cu") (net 23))
 (segment (start 96.8 95.2) (end 99.1 97.5) (width 0.2) (layer "B.Cu") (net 23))
 (segment (start 99.1 97.5) (end 107.9329 97.5) (width 0.2) (layer "B.Cu") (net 23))
 (segment (start 110.4329 95) (end 110.5 95) (width 0.2) (layer "B.Cu") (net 23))
 (segment (start 109 94.5) (end 110.5 94.5) (width 0.2) (layer "B.Cu") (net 22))
 (segment (start 101 95.2) (end 108.3 95.2) (width 0.2) (layer "B.Cu") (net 22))
 (segment (start 108.3 95.2) (end 109 94.5) (width 0.2) (layer "B.Cu") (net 22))
 (segment (start 86.5 84) (end 79.5 91) (width 0.2) (layer "F.Cu") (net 5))
 (segment (start 93.451 83.051) (end 92.502 84) (width 0.2) (layer "F.Cu") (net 5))
 (segment (start 94.12524 81.349) (end 93.451 82.02324) (width 0.2) (layer "F.Cu") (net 5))
 (segment (start 88.539999 114.54) (end 92.25 114.54) (width 0.2) (layer "F.Cu") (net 5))
 (segment (start 99.92 82.5) (end 98.769 81.349) (width 0.2) (layer "F.Cu") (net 5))
 (segment (start 93.451 82.02324) (end 93.451 83.051) (width 0.2) (layer "F.Cu") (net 5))
 (segment (start 79.5 91) (end 79.5 105.500001) (width 0.2) (layer "F.Cu") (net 5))
 (segment (start 98.769 81.349) (end 94.12524 81.349) (width 0.2) (layer "F.Cu") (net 5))
 (segment (start 79.5 105.500001) (end 88.539999 114.54) (width 0.2) (layer "F.Cu") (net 5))
 (segment (start 92.502 84) (end 86.5 84) (width 0.2) (layer "F.Cu") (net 5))
 (segment (start 107.57776 126) (end 109.5 124.07776) (width 0.2) (layer "B.Cu") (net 14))
 (segment (start 109.5 124.07776) (end 109.5 96.5) (width 0.2) (layer "B.Cu") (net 14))
 (segment (start 109.5 96.5) (end 110.5 95.5) (width 0.2) (layer "B.Cu") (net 14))
 (segment (start 92.25 127.24) (end 93.49 126) (width 0.2) (layer "B.Cu") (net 14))
 (segment (start 93.49 126) (end 107.57776 126) (width 0.2) (layer "B.Cu") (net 14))
 (segment (start 107.25 127.24) (end 110.03355 124.45645) (width 0.2) (layer "B.Cu") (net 11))
 (segment (start 111 95.5671) (end 111 94.5) (width 0.2) (layer "B.Cu") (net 11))
 (segment (start 110.853553 95.713547) (end 111 95.5671) (width 0.2) (layer "B.Cu") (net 11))
 (segment (start 110.03355 96.53355) (end 110.853553 95.713547) (width 0.2) (layer "B.Cu") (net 11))
 (segment (start 110.03355 124.45645) (end 110.03355 96.53355) (width 0.2) (layer "B.Cu") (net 11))
 (segment (start 97.667133 86.198) (end 107.670678 86.198) (width 0.2) (layer "B.Cu") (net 19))
 (segment (start 107.670678 86.198) (end 110.5 89.027322) (width 0.2) (layer "B.Cu") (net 19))
 (segment (start 98 106.2) (end 95.149 103.349) (width 0.2) (layer "B.Cu") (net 19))
 (segment (start 95.149 88.716133) (end 97.667133 86.198) (width 0.2) (layer "B.Cu") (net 19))
 (segment (start 110.5 89.027322) (end 110.5 93) (width 0.2) (layer "B.Cu") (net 19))
 (segment (start 95.149 103.349) (end 95.149 88.716133) (width 0.2) (layer "B.Cu") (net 19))
 (segment (start 111 88.960222) (end 111 92.5) (width 0.2) (layer "B.Cu") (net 17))
 (segment (start 107.836778 85.797) (end 111 88.960222) (width 0.2) (layer "B.Cu") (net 17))
 (segment (start 111 92.5) (end 111 93) (width 0.2) (layer "B.Cu") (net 17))
 (segment (start 94.748 88.550033) (end 97.501033 85.797) (width 0.2) (layer "B.Cu") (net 17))
 (segment (start 92.5 106.2) (end 94.748 103.952) (width 0.2) (layer "B.Cu") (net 17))
 (segment (start 94.748 103.952) (end 94.748 88.550033) (width 0.2) (layer "B.Cu") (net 17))
 (segment (start 97.501033 85.797) (end 107.836778 85.797) (width 0.2) (layer "B.Cu") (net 17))
 (segment (start 94.251 100.249) (end 94.251 88.479933) (width 0.2) (layer "B.Cu") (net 18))
 (segment (start 111.401 93.1661) (end 111.0671 93.5) (width 0.2) (layer "B.Cu") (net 18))
 (segment (start 97.334933 85.396) (end 108.002878 85.396) (width 0.2) (layer "B.Cu") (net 18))
 (segment (start 111.0671 93.5) (end 111 93.5) (width 0.2) (layer "B.Cu") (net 18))
 (segment (start 108.002878 85.396) (end 111.401 88.794122) (width 0.2) (layer "B.Cu") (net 18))
 (segment (start 92.5 102) (end 94.251 100.249) (width 0.2) (layer "B.Cu") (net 18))
 (segment (start 94.251 88.479933) (end 97.334933 85.396) (width 0.2) (layer "B.Cu") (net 18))
 (segment (start 111.401 88.794122) (end 111.401 93.1661) (width 0.2) (layer "B.Cu") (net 18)))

